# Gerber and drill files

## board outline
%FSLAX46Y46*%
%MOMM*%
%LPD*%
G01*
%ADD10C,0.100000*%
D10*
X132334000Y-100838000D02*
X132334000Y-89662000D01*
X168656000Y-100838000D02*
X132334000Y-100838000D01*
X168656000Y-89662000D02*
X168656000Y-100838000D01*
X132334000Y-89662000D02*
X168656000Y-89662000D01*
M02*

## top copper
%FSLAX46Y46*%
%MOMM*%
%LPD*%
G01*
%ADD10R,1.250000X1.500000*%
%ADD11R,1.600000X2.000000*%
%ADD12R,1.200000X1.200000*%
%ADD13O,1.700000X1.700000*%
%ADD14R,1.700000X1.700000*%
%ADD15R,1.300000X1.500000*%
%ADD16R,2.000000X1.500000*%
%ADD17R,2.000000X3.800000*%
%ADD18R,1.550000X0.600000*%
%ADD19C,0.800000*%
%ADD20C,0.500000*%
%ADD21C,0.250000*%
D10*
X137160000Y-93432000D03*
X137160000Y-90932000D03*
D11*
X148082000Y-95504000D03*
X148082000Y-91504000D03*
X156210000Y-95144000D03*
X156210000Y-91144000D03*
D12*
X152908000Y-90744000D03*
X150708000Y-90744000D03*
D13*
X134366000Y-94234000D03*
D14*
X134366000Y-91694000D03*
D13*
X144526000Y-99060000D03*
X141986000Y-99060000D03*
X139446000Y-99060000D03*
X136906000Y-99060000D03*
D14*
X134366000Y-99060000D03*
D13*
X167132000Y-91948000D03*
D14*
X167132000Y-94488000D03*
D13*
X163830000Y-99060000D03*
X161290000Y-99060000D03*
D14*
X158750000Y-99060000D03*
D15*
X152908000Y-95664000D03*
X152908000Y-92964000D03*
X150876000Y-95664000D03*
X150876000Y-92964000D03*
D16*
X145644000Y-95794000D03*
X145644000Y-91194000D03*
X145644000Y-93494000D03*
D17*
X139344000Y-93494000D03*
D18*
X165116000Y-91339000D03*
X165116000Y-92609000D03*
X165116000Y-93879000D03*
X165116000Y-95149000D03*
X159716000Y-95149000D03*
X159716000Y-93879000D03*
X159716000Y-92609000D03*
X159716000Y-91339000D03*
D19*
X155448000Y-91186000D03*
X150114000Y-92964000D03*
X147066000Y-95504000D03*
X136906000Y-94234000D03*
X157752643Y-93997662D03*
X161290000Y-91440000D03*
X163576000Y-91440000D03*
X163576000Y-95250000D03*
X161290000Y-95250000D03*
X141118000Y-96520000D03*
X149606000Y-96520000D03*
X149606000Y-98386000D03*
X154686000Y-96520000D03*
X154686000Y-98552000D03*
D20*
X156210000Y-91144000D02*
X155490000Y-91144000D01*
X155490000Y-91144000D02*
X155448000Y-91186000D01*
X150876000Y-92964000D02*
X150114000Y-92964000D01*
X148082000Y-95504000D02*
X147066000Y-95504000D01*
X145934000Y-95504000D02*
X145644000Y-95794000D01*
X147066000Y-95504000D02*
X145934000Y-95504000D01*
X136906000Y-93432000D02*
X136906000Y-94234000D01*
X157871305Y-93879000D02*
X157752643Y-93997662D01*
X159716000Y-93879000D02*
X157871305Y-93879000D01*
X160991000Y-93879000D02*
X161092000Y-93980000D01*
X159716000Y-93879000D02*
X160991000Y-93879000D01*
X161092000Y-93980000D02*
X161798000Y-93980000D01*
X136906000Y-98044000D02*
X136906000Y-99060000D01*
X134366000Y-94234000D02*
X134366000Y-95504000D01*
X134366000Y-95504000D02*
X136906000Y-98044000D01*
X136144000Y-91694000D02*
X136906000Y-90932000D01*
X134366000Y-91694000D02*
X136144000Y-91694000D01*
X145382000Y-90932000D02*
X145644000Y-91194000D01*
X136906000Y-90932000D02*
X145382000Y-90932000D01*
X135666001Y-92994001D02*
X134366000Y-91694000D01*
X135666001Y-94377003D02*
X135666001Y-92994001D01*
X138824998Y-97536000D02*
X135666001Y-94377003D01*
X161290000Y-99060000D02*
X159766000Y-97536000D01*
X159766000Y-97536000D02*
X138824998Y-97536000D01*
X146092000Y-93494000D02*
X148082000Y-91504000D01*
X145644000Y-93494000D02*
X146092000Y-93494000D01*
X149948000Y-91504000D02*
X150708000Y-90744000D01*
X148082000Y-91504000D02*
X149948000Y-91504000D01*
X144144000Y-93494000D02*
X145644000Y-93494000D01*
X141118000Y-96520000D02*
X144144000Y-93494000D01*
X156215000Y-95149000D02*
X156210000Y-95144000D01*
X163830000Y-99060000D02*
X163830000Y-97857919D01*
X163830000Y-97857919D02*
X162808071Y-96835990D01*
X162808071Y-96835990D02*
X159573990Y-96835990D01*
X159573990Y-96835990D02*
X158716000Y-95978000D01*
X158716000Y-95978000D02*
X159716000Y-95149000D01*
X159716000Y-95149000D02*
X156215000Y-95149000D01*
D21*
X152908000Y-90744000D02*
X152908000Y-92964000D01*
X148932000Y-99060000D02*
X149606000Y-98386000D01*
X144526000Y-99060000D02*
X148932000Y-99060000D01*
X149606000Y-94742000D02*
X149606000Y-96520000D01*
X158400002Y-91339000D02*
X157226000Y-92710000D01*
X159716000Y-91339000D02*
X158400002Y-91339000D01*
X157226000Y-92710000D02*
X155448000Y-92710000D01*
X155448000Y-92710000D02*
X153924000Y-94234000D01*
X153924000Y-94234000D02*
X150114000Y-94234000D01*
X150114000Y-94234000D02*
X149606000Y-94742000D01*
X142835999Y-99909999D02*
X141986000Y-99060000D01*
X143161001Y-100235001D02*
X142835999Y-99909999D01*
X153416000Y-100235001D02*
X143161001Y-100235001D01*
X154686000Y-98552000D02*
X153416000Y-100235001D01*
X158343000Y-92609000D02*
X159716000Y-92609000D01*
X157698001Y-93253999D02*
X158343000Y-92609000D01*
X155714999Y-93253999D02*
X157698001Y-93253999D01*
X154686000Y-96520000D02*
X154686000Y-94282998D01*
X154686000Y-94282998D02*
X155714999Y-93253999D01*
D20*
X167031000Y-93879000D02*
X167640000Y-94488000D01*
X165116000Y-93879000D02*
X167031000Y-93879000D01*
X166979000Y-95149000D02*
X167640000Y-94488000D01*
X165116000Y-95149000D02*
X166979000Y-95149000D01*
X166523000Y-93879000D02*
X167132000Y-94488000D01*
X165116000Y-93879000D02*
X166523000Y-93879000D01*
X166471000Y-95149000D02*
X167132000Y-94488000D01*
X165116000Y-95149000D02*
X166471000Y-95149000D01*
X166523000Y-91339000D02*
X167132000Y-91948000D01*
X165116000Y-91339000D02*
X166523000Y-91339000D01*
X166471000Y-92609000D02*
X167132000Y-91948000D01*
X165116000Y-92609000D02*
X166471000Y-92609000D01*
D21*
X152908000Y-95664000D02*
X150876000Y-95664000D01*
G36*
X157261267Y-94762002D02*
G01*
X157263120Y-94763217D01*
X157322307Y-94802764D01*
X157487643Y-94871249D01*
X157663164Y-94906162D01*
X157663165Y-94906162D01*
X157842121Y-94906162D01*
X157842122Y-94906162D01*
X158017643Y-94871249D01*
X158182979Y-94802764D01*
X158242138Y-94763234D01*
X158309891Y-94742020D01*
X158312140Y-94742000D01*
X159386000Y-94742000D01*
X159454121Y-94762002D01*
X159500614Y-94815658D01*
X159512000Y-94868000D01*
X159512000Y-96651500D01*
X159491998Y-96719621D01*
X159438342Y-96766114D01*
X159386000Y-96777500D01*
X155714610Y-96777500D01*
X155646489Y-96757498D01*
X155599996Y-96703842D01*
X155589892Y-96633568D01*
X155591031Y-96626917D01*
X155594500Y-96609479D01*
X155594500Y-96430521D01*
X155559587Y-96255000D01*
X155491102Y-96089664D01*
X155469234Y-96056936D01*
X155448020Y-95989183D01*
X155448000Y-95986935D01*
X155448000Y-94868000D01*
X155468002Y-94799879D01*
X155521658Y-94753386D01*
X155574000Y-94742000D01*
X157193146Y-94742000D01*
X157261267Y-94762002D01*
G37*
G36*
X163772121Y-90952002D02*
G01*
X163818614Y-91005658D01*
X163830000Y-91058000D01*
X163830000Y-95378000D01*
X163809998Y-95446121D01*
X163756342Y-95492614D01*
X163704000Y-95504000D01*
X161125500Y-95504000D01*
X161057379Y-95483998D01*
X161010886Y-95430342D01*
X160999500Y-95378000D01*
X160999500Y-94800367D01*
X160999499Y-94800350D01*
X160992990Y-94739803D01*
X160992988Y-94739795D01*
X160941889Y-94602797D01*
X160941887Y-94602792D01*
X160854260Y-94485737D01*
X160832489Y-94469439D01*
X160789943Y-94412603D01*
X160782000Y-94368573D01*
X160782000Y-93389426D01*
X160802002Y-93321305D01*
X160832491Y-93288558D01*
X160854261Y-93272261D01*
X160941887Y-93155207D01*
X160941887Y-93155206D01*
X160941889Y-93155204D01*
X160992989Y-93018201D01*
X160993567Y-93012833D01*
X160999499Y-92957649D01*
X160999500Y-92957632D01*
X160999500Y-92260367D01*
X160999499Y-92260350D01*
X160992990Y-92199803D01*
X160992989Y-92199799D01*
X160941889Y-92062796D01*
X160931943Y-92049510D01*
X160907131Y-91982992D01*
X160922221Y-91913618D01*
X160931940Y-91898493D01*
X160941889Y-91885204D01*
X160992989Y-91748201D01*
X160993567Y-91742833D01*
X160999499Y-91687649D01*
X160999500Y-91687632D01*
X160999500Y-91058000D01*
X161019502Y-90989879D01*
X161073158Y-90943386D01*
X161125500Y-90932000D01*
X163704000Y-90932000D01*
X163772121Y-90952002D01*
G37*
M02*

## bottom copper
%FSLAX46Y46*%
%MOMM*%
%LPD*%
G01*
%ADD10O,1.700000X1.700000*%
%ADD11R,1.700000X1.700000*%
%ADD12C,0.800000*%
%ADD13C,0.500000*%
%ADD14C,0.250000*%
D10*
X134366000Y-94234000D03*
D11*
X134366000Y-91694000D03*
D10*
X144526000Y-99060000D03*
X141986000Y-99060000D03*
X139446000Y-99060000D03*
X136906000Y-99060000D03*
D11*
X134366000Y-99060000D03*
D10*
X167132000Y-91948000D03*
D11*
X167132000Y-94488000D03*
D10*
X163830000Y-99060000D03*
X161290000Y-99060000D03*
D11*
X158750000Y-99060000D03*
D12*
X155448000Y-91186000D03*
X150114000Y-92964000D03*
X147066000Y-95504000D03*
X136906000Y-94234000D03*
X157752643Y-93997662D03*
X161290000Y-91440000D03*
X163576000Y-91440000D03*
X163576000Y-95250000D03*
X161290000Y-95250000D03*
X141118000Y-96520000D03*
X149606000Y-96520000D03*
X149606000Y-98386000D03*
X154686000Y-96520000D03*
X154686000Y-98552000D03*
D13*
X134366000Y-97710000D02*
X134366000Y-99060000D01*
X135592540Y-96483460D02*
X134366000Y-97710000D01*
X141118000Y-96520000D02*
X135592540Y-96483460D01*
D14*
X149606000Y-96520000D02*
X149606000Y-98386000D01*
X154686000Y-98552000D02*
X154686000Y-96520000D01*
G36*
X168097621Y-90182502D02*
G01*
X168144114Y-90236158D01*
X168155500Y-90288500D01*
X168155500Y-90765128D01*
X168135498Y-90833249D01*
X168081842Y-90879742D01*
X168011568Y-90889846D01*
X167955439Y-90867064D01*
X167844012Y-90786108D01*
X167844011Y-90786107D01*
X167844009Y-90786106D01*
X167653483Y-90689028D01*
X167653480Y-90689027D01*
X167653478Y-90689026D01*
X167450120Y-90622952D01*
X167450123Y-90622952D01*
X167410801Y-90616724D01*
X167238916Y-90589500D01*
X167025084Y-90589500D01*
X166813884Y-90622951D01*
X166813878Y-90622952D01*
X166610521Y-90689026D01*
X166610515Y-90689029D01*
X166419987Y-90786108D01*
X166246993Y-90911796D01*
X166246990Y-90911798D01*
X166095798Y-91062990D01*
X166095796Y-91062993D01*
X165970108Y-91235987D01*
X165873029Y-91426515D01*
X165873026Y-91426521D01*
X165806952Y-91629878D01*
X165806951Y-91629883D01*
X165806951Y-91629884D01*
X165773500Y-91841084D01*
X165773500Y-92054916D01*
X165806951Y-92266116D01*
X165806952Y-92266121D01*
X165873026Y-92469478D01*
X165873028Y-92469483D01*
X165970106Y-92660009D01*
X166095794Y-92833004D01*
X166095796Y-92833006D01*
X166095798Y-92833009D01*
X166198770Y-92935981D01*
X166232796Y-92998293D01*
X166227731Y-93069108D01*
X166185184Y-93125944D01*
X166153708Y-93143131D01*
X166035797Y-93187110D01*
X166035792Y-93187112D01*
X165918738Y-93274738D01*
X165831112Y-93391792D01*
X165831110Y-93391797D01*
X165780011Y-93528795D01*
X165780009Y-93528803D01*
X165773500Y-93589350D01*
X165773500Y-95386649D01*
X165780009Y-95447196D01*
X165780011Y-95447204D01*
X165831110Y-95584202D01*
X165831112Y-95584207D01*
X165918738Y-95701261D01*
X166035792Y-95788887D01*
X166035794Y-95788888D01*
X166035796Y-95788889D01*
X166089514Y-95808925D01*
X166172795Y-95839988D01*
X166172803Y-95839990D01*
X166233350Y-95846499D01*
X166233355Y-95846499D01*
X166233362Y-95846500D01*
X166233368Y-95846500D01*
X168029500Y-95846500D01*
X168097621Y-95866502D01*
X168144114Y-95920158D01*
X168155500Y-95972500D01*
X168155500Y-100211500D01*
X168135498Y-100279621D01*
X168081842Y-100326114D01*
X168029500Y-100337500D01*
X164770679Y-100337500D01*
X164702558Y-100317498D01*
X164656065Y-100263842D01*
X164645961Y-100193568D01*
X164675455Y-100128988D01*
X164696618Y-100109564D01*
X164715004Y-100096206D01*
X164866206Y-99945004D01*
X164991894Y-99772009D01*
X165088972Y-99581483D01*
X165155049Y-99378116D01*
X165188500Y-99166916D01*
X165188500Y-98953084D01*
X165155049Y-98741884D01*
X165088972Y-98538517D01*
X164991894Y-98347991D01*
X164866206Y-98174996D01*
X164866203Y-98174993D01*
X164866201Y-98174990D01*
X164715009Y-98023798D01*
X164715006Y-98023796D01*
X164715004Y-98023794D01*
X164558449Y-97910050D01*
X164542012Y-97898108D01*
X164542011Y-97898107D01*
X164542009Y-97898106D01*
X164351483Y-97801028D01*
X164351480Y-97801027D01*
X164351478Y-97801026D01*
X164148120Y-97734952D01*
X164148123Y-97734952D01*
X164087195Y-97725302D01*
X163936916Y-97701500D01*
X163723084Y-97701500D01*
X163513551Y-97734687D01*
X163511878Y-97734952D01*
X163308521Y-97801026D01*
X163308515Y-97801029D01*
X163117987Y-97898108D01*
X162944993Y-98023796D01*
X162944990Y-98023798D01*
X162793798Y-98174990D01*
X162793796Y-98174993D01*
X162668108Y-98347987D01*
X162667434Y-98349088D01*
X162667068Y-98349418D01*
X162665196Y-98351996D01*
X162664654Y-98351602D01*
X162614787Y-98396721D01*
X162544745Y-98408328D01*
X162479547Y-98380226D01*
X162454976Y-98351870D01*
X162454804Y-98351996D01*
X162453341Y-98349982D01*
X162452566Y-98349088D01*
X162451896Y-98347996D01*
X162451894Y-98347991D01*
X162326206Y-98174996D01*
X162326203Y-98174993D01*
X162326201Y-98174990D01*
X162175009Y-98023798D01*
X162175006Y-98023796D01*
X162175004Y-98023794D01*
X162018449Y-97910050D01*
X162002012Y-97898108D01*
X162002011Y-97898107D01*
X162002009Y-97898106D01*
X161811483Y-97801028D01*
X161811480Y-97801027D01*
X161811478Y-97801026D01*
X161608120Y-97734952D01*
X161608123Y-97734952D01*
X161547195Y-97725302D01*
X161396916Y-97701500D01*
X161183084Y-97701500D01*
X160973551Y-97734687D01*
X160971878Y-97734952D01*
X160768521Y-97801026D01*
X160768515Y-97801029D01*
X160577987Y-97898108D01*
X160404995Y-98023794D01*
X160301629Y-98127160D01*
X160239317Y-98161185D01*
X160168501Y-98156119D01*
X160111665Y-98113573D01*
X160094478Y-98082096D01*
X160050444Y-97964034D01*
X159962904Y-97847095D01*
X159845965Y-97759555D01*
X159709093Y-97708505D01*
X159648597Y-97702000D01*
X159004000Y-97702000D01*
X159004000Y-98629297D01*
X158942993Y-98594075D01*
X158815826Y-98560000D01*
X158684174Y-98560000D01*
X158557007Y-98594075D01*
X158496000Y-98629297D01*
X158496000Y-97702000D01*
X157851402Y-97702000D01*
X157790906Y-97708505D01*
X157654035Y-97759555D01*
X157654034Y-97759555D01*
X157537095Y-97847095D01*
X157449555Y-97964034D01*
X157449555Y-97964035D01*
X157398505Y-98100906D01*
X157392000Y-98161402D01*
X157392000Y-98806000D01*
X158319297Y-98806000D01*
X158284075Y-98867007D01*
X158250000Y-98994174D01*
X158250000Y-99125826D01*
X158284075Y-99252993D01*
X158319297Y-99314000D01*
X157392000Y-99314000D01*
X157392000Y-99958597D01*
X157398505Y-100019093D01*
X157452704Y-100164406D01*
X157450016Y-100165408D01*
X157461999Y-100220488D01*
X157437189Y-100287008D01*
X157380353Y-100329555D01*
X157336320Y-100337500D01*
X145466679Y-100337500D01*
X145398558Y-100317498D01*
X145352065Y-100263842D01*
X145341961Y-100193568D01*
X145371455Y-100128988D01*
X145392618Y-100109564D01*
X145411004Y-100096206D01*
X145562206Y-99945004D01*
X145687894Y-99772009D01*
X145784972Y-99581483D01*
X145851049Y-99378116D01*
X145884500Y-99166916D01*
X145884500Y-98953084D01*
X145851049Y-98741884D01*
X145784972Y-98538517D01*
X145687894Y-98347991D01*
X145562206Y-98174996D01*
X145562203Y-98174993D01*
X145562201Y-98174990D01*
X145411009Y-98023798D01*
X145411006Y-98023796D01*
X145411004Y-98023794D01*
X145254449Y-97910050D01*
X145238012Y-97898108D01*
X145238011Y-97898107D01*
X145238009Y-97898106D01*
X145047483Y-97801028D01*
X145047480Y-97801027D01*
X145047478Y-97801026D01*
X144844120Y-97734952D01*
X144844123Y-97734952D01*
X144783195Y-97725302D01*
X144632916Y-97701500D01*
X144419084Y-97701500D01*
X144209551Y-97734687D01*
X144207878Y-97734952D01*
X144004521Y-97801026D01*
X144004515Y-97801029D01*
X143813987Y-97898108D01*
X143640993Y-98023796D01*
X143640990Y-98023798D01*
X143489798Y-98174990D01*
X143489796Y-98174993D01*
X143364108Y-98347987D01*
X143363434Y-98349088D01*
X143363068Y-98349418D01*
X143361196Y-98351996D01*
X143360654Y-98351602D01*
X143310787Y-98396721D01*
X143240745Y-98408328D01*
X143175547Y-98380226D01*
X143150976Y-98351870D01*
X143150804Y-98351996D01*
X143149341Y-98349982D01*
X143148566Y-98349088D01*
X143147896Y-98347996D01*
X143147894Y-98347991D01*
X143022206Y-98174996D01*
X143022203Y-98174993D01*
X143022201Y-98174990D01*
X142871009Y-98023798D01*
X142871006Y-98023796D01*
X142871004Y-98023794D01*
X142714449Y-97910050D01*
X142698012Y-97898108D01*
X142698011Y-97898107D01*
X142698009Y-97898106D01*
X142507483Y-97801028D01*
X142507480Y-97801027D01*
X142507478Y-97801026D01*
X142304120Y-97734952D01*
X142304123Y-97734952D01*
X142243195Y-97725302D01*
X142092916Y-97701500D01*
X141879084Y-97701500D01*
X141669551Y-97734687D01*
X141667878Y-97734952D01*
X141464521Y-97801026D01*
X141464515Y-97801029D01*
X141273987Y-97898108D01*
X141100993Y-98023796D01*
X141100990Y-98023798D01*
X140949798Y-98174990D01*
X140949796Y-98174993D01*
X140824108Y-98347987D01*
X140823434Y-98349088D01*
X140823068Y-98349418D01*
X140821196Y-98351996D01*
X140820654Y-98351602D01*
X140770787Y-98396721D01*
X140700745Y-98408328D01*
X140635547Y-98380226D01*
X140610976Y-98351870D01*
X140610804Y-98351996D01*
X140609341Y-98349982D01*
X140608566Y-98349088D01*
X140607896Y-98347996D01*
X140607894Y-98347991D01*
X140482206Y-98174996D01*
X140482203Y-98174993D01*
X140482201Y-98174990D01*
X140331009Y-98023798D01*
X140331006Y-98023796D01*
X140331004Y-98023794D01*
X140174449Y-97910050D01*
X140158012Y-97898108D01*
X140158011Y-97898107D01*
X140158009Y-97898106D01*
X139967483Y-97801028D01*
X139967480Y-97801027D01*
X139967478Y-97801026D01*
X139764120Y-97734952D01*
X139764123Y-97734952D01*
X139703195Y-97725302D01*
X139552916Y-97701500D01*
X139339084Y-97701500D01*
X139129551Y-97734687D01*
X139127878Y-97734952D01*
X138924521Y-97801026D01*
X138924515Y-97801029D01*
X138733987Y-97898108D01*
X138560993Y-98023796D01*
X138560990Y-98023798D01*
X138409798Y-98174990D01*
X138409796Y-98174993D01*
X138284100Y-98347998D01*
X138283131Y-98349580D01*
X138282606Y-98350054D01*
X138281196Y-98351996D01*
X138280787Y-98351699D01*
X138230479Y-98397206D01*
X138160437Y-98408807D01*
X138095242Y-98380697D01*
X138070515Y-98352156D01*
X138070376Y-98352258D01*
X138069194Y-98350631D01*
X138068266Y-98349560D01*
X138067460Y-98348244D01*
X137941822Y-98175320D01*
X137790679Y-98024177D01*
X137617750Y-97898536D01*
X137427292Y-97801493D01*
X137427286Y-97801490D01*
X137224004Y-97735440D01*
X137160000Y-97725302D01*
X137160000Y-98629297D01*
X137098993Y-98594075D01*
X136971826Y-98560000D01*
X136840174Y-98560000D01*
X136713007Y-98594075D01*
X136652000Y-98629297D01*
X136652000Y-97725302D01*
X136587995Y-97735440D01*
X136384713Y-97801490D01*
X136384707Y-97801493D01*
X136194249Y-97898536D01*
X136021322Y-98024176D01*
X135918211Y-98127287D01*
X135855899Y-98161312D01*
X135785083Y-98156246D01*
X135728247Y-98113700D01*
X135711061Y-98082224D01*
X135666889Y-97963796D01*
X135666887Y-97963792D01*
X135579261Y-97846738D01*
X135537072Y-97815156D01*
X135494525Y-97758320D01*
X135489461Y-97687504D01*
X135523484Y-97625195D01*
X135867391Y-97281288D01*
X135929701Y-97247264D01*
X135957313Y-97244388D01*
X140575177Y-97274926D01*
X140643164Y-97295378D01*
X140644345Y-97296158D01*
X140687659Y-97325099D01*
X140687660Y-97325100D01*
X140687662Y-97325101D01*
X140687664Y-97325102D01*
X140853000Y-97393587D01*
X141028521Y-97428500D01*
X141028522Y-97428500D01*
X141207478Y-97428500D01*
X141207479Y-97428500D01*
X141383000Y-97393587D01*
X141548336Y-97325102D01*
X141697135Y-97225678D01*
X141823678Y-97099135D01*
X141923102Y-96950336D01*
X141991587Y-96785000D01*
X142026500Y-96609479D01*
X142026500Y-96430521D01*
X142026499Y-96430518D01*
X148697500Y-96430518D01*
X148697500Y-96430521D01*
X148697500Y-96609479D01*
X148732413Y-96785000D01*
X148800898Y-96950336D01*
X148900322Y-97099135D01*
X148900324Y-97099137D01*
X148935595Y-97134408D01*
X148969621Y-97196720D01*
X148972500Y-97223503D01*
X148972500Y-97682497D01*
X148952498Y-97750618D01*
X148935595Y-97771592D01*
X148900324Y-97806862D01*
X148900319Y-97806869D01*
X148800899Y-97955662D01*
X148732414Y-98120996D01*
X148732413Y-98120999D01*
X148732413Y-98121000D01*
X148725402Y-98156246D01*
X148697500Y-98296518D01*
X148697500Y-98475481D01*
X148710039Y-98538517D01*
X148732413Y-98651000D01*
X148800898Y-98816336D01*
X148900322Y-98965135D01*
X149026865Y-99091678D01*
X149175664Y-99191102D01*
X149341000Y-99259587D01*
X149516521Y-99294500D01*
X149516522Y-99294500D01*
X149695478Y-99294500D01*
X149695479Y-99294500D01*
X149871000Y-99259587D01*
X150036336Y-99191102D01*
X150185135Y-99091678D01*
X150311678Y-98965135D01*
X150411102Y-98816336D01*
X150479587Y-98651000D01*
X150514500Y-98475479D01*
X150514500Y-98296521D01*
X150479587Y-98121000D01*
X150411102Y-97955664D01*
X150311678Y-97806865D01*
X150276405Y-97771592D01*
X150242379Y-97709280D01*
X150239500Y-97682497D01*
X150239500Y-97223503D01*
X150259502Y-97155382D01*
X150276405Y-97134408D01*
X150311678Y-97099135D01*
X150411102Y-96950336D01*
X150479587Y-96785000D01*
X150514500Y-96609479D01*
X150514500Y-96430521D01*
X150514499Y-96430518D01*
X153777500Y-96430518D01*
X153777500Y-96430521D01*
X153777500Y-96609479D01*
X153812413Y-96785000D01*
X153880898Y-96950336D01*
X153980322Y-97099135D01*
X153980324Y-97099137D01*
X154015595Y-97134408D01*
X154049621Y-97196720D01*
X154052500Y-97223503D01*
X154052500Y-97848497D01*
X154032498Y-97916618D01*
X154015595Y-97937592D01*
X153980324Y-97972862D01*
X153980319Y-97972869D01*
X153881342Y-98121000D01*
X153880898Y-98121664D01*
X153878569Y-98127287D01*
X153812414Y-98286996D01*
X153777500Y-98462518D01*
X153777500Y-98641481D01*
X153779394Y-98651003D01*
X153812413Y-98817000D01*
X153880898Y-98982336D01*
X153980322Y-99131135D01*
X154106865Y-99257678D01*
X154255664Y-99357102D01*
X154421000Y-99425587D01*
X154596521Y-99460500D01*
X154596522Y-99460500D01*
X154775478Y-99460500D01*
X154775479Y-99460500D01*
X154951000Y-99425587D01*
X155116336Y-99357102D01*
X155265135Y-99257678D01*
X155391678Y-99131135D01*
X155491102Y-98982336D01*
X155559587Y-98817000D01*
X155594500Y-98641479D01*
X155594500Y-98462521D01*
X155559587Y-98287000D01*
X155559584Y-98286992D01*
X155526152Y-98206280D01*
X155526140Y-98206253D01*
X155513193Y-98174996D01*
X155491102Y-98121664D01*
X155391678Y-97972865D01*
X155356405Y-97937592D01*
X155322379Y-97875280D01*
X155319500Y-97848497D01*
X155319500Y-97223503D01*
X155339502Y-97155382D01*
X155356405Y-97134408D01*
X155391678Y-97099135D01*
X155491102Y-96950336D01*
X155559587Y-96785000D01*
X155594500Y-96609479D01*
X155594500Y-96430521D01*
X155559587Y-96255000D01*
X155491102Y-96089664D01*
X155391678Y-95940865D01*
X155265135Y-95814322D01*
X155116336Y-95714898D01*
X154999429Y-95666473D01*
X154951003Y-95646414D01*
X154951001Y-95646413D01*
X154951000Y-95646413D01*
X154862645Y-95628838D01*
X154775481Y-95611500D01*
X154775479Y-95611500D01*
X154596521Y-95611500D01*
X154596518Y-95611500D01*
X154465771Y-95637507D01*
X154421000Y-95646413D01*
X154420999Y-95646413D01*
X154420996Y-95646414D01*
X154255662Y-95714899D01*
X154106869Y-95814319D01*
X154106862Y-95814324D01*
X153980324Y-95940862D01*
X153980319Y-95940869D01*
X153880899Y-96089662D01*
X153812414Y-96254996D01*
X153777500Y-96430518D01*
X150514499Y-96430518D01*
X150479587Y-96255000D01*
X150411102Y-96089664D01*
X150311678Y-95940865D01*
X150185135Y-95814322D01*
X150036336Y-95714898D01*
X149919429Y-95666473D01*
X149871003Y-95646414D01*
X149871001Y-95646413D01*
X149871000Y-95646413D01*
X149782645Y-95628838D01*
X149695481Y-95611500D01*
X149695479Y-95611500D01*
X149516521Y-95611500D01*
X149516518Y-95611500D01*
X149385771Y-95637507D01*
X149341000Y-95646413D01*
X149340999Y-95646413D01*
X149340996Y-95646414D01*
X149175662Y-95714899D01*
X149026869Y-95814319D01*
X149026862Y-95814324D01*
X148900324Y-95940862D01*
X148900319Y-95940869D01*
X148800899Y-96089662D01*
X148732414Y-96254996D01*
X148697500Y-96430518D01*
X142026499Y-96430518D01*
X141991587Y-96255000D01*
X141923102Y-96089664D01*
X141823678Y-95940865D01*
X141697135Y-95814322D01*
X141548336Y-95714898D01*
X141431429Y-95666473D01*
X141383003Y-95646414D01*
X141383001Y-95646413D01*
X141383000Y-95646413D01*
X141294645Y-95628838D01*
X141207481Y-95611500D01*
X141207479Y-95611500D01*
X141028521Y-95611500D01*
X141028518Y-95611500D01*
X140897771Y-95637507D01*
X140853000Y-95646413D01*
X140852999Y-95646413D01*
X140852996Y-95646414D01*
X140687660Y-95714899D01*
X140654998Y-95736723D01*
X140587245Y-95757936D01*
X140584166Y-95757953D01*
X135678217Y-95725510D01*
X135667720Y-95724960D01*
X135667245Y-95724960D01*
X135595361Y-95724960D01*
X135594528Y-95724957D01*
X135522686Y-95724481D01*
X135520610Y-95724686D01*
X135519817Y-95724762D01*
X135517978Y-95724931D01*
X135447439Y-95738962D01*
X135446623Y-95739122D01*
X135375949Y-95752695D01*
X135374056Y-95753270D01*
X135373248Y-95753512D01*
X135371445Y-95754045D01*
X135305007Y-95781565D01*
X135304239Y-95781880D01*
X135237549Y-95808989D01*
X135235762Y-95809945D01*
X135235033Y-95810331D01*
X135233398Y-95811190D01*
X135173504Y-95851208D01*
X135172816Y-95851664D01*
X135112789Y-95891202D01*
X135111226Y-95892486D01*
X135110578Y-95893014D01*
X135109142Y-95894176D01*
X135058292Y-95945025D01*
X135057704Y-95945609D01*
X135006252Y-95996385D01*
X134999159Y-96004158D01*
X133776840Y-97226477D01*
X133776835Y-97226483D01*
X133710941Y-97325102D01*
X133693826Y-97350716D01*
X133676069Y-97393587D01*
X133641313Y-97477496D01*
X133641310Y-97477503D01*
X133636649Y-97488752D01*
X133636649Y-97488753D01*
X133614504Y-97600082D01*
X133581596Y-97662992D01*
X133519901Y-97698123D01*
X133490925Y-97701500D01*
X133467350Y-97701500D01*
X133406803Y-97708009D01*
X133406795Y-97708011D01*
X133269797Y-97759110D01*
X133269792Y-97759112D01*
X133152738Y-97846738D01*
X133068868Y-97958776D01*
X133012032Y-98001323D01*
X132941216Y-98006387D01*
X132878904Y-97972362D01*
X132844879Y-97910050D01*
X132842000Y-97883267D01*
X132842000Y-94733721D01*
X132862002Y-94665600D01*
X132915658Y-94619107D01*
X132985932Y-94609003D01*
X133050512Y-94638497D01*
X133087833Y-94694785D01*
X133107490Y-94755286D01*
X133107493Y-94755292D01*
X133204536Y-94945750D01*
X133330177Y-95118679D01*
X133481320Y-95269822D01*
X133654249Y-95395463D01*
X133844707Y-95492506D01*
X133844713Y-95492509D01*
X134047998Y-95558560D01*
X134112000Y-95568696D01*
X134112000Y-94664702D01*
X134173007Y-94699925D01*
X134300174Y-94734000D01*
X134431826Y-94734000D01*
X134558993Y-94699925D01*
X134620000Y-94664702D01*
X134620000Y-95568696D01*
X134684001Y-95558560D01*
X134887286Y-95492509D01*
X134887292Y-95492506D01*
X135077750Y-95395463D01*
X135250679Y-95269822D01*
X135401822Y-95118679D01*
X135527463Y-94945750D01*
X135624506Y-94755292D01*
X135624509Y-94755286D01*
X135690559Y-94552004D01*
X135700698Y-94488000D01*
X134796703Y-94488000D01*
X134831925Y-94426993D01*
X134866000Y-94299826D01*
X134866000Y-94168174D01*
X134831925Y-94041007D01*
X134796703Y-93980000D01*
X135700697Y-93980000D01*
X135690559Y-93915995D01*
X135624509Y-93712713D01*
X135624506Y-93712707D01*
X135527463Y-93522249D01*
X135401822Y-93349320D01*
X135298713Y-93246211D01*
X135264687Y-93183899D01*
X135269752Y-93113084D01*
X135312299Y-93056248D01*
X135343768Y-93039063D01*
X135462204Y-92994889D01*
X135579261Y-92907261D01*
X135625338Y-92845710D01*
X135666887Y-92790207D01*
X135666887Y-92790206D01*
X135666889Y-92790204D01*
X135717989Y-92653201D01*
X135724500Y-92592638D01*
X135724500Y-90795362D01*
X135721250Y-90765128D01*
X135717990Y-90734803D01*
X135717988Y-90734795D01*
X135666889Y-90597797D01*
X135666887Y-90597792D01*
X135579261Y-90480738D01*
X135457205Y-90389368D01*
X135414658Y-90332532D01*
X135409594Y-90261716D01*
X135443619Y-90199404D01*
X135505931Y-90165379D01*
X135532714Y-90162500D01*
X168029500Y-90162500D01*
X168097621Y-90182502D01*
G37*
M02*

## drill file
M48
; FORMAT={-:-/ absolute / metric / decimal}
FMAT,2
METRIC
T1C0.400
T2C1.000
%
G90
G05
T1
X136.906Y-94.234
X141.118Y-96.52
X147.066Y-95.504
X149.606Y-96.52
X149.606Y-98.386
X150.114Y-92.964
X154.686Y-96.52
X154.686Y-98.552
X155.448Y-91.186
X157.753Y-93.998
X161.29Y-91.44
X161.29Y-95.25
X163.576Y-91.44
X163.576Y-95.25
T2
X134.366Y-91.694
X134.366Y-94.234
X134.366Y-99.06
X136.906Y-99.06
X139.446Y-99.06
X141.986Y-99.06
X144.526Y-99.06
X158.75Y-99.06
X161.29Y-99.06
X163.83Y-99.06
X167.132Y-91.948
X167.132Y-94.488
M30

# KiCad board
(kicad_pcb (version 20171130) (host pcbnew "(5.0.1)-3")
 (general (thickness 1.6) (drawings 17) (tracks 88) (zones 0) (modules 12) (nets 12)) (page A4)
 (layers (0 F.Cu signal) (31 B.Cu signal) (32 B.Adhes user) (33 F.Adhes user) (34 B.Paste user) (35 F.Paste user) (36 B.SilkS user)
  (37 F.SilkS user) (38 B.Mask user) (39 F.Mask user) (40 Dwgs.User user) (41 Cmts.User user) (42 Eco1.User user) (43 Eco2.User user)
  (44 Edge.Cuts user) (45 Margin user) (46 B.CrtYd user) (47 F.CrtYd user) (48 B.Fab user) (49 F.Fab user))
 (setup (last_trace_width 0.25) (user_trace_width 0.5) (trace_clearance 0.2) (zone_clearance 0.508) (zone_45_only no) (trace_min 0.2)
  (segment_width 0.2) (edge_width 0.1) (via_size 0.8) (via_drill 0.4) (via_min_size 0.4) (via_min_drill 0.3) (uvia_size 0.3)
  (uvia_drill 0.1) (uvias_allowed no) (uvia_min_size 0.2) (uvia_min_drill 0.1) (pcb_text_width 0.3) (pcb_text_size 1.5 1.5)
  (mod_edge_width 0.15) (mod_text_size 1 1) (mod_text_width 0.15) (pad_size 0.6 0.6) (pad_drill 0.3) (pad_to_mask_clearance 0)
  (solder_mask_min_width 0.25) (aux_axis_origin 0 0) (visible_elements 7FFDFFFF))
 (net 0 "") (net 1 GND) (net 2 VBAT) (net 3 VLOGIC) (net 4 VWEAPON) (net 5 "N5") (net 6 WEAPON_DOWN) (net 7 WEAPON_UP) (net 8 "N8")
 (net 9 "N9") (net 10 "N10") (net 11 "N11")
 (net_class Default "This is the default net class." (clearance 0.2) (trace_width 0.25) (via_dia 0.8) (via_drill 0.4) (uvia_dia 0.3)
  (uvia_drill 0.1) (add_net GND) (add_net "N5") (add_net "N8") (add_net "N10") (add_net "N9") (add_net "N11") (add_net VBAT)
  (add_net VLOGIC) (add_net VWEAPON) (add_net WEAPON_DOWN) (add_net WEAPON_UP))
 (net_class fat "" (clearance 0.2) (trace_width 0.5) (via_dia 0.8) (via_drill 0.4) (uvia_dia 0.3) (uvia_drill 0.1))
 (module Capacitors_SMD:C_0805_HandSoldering (layer F.Cu) (at 137.16 92.182 270)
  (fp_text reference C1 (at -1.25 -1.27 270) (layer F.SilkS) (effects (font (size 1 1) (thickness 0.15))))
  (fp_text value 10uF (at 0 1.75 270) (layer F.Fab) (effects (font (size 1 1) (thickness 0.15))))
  (pad 2 smd rect (at 1.25 0 270) (size 1.5 1.25) (layers F.Cu F.Paste F.Mask) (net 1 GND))
  (pad 1 smd rect (at -1.25 0 270) (size 1.5 1.25) (layers F.Cu F.Paste F.Mask) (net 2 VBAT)))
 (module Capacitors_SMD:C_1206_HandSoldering (layer F.Cu) (at 148.082 93.504 270)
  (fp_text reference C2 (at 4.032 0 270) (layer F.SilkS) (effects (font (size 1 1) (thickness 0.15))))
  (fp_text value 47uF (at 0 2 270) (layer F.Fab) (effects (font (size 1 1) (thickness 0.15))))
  (pad 2 smd rect (at 2 0 270) (size 2 1.6) (layers F.Cu F.Paste F.Mask) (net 1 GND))
  (pad 1 smd rect (at -2 0 270) (size 2 1.6) (layers F.Cu F.Paste F.Mask) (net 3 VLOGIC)))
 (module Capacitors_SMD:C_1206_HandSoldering (layer F.Cu) (at 156.21 93.144 90)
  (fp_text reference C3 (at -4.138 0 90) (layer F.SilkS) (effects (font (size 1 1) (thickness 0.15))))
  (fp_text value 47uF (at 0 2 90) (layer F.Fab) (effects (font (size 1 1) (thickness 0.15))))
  (pad 1 smd rect (at -2 0 90) (size 2 1.6) (layers F.Cu F.Paste F.Mask) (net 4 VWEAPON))
  (pad 2 smd rect (at 2 0 90) (size 2 1.6) (layers F.Cu F.Paste F.Mask) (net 1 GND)))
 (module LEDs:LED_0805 (layer F.Cu) (at 151.808 90.744 180)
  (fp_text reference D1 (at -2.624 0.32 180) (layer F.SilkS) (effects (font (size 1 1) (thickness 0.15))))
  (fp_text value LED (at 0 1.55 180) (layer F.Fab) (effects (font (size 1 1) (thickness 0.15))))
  (pad 1 smd rect (at -1.1 0) (size 1.2 1.2) (layers F.Cu F.Paste F.Mask) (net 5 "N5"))
  (pad 2 smd rect (at 1.1 0) (size 1.2 1.2) (layers F.Cu F.Paste F.Mask) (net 3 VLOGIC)))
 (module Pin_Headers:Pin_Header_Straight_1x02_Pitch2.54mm (layer F.Cu) (at 134.366 91.694)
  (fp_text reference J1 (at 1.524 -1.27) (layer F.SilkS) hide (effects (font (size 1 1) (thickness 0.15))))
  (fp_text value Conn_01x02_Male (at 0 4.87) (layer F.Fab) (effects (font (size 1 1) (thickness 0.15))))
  (pad 2 thru_hole oval (at 0 2.54) (size 1.7 1.7) (drill 1) (layers *.Cu *.Mask) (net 1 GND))
  (pad 1 thru_hole rect (at 0 0) (size 1.7 1.7) (drill 1) (layers *.Cu *.Mask) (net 2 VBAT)))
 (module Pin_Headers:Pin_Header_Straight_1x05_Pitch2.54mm (layer F.Cu) (at 134.366 99.06 90)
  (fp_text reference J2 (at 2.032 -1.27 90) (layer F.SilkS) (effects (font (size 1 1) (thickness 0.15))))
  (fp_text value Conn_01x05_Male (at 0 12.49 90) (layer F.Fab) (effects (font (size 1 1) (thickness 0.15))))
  (pad 5 thru_hole oval (at 0 10.16 90) (size 1.7 1.7) (drill 1) (layers *.Cu *.Mask) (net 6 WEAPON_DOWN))
  (pad 4 thru_hole oval (at 0 7.62 90) (size 1.7 1.7) (drill 1) (layers *.Cu *.Mask) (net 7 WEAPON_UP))
  (pad 3 thru_hole oval (at 0 5.08 90) (size 1.7 1.7) (drill 1) (layers *.Cu *.Mask) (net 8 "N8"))
  (pad 2 thru_hole oval (at 0 2.54 90) (size 1.7 1.7) (drill 1) (layers *.Cu *.Mask) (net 1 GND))
  (pad 1 thru_hole rect (at 0 0 90) (size 1.7 1.7) (drill 1) (layers *.Cu *.Mask) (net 3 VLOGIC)))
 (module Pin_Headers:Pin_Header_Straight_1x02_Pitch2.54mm (layer F.Cu) (at 167.132 94.488 180)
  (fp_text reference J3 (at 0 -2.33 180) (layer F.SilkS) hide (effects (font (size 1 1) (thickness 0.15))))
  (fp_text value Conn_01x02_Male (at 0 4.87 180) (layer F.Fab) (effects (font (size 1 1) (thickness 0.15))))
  (pad 2 thru_hole oval (at 0 2.54 180) (size 1.7 1.7) (drill 1) (layers *.Cu *.Mask) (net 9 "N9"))
  (pad 1 thru_hole rect (at 0 0 180) (size 1.7 1.7) (drill 1) (layers *.Cu *.Mask) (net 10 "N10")))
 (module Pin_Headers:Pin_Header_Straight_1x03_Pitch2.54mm (layer F.Cu) (at 158.75 99.06 90)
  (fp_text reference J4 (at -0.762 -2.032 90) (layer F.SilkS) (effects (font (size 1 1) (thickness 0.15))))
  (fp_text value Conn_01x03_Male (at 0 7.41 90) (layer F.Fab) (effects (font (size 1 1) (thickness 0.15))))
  (pad 3 thru_hole oval (at 0 5.08 90) (size 1.7 1.7) (drill 1) (layers *.Cu *.Mask) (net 4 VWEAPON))
  (pad 2 thru_hole oval (at 0 2.54 90) (size 1.7 1.7) (drill 1) (layers *.Cu *.Mask) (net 2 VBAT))
  (pad 1 thru_hole rect (at 0 0 90) (size 1.7 1.7) (drill 1) (layers *.Cu *.Mask) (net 1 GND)))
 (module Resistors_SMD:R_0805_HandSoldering (layer F.Cu) (at 152.908 94.314 270)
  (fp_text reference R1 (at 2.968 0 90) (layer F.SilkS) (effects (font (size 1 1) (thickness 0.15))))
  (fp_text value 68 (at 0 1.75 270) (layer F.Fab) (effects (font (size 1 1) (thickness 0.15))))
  (pad 2 smd rect (at 1.35 0 270) (size 1.5 1.3) (layers F.Cu F.Paste F.Mask) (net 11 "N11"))
  (pad 1 smd rect (at -1.35 0 270) (size 1.5 1.3) (layers F.Cu F.Paste F.Mask) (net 5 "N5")))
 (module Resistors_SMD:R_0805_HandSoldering (layer F.Cu) (at 150.876 94.314 90)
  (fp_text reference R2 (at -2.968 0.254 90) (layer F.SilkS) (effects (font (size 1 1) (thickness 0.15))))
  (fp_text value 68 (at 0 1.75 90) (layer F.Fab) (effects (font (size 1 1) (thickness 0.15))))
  (pad 1 smd rect (at -1.35 0 90) (size 1.5 1.3) (layers F.Cu F.Paste F.Mask) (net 11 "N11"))
  (pad 2 smd rect (at 1.35 0 90) (size 1.5 1.3) (layers F.Cu F.Paste F.Mask) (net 1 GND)))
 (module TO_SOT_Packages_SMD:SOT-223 (layer F.Cu) (at 142.494 93.494 180)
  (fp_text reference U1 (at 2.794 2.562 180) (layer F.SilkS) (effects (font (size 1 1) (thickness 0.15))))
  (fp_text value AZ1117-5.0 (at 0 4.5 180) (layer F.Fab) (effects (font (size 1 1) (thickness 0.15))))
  (pad 1 smd rect (at -3.15 -2.3 180) (size 2 1.5) (layers F.Cu F.Paste F.Mask) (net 1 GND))
  (pad 3 smd rect (at -3.15 2.3 180) (size 2 1.5) (layers F.Cu F.Paste F.Mask) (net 2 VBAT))
  (pad 2 smd rect (at -3.15 0 180) (size 2 1.5) (layers F.Cu F.Paste F.Mask) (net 3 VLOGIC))
  (pad 4 smd rect (at 3.15 0 180) (size 2 3.8) (layers F.Cu F.Paste F.Mask)))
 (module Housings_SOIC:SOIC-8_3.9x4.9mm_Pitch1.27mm (layer F.Cu) (at 162.416 93.244)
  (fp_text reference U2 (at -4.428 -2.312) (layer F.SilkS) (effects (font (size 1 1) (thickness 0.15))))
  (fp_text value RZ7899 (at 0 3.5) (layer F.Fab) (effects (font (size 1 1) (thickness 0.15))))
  (pad 8 smd rect (at 2.7 -1.905) (size 1.55 0.6) (layers F.Cu F.Paste F.Mask) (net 9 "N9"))
  (pad 7 smd rect (at 2.7 -0.635) (size 1.55 0.6) (layers F.Cu F.Paste F.Mask) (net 9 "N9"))
  (pad 6 smd rect (at 2.7 0.635) (size 1.55 0.6) (layers F.Cu F.Paste F.Mask) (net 10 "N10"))
  (pad 5 smd rect (at 2.7 1.905) (size 1.55 0.6) (layers F.Cu F.Paste F.Mask) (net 10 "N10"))
  (pad 4 smd rect (at -2.7 1.905) (size 1.55 0.6) (layers F.Cu F.Paste F.Mask) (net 4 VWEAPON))
  (pad 3 smd rect (at -2.7 0.635) (size 1.55 0.6) (layers F.Cu F.Paste F.Mask) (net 1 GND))
  (pad 2 smd rect (at -2.7 -0.635) (size 1.55 0.6) (layers F.Cu F.Paste F.Mask) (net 7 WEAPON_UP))
  (pad 1 smd rect (at -2.7 -1.905) (size 1.55 0.6) (layers F.Cu F.Paste F.Mask) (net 6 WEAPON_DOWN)))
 (gr_line (start 132.334 100.838) (end 132.334 89.662) (layer Edge.Cuts) (width 0.1))
 (gr_line (start 168.656 100.838) (end 132.334 100.838) (layer Edge.Cuts) (width 0.1))
 (gr_line (start 168.656 89.662) (end 168.656 100.838) (layer Edge.Cuts) (width 0.1))
 (gr_line (start 132.334 89.662) (end 168.656 89.662) (layer Edge.Cuts) (width 0.1))
 (via (at 155.448 91.186) (size 0.8) (drill 0.4) (layers F.Cu B.Cu) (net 1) (status 30))
 (segment (start 156.21 91.144) (end 155.49 91.144) (width 0.5) (layer F.Cu) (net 1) (status 30))
 (segment (start 155.49 91.144) (end 155.448 91.186) (width 0.5) (layer F.Cu) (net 1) (status 30))
 (via (at 150.114 92.964) (size 0.8) (drill 0.4) (layers F.Cu B.Cu) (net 1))
 (segment (start 150.876 92.964) (end 150.114 92.964) (width 0.5) (layer F.Cu) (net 1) (status 10))
 (via (at 147.066 95.504) (size 0.8) (drill 0.4) (layers F.Cu B.Cu) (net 1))
 (segment (start 148.082 95.504) (end 147.066 95.504) (width 0.5) (layer F.Cu) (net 1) (status 10))
 (segment (start 145.934 95.504) (end 145.644 95.794) (width 0.5) (layer F.Cu) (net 1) (status 30))
 (segment (start 147.066 95.504) (end 145.934 95.504) (width 0.5) (layer F.Cu) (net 1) (status 20))
 (via (at 136.906 94.234) (size 0.8) (drill 0.4) (layers F.Cu B.Cu) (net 1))
 (segment (start 136.906 93.432) (end 136.906 94.234) (width 0.5) (layer F.Cu) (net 1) (status 10))
 (via (at 157.752643 93.997662) (size 0.8) (drill 0.4) (layers F.Cu B.Cu) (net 1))
 (segment (start 157.871305 93.879) (end 157.752643 93.997662) (width 0.5) (layer F.Cu) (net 1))
 (segment (start 159.716 93.879) (end 157.871305 93.879) (width 0.5) (layer F.Cu) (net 1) (status 10))
 (segment (start 160.991 93.879) (end 161.092 93.98) (width 0.5) (layer F.Cu) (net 1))
 (segment (start 159.716 93.879) (end 160.991 93.879) (width 0.5) (layer F.Cu) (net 1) (status 10))
 (segment (start 161.092 93.98) (end 161.798 93.98) (width 0.5) (layer F.Cu) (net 1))
 (via (at 161.29 91.44) (size 0.8) (drill 0.4) (layers F.Cu B.Cu) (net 1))
 (via (at 163.576 91.44) (size 0.8) (drill 0.4) (layers F.Cu B.Cu) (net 1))
 (via (at 163.576 95.25) (size 0.8) (drill 0.4) (layers F.Cu B.Cu) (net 1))
 (via (at 161.29 95.25) (size 0.8) (drill 0.4) (layers F.Cu B.Cu) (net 1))
 (segment (start 136.906 98.044) (end 136.906 99.06) (width 0.5) (layer F.Cu) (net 1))
 (segment (start 134.366 94.234) (end 134.366 95.504) (width 0.5) (layer F.Cu) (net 1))
 (segment (start 134.366 95.504) (end 136.906 98.044) (width 0.5) (layer F.Cu) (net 1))
 (segment (start 136.144 91.694) (end 136.906 90.932) (width 0.5) (layer F.Cu) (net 2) (status 20))
 (segment (start 134.366 91.694) (end 136.144 91.694) (width 0.5) (layer F.Cu) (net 2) (status 10))
 (segment (start 145.382 90.932) (end 145.644 91.194) (width 0.5) (layer F.Cu) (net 2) (status 30))
 (segment (start 136.906 90.932) (end 145.382 90.932) (width 0.5) (layer F.Cu) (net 2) (status 30))
 (segment (start 135.666001 92.994001) (end 134.366 91.694) (width 0.5) (layer F.Cu) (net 2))
 (segment (start 135.666001 94.377003) (end 135.666001 92.994001) (width 0.5) (layer F.Cu) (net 2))
 (segment (start 138.824998 97.536) (end 135.666001 94.377003) (width 0.5) (layer F.Cu) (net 2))
 (segment (start 161.29 99.06) (end 159.766 97.536) (width 0.5) (layer F.Cu) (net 2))
 (segment (start 159.766 97.536) (end 138.824998 97.536) (width 0.5) (layer F.Cu) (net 2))
 (segment (start 146.092 93.494) (end 148.082 91.504) (width 0.5) (layer F.Cu) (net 3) (status 30))
 (segment (start 145.644 93.494) (end 146.092 93.494) (width 0.5) (layer F.Cu) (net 3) (status 30))
 (segment (start 149.948 91.504) (end 150.708 90.744) (width 0.5) (layer F.Cu) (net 3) (status 20))
 (segment (start 148.082 91.504) (end 149.948 91.504) (width 0.5) (layer F.Cu) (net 3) (status 10))
 (segment (start 134.366 97.71) (end 134.366 99.06) (width 0.5) (layer B.Cu) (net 3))
 (segment (start 135.59254 96.48346) (end 134.366 97.71) (width 0.5) (layer B.Cu) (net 3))
 (segment (start 141.118 96.52) (end 135.59254 96.48346) (width 0.5) (layer B.Cu) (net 3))
 (via (at 141.118 96.52) (size 0.8) (drill 0.4) (layers F.Cu B.Cu) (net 3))
 (segment (start 144.144 93.494) (end 145.644 93.494) (width 0.5) (layer F.Cu) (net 3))
 (segment (start 141.118 96.52) (end 144.144 93.494) (width 0.5) (layer F.Cu) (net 3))
 (segment (start 156.215 95.149) (end 156.21 95.144) (width 0.5) (layer F.Cu) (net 4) (status 30))
 (segment (start 163.83 99.06) (end 163.83 97.857919) (width 0.5) (layer F.Cu) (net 4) (status 10))
 (segment (start 163.83 97.857919) (end 162.808071 96.83599) (width 0.5) (layer F.Cu) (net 4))
 (segment (start 162.808071 96.83599) (end 159.57399 96.83599) (width 0.5) (layer F.Cu) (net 4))
 (segment (start 159.57399 96.83599) (end 158.716 95.978) (width 0.5) (layer F.Cu) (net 4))
 (segment (start 158.716 95.978) (end 159.716 95.149) (width 0.5) (layer F.Cu) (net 4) (status 20))
 (segment (start 159.716 95.149) (end 156.215 95.149) (width 0.5) (layer F.Cu) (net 4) (status 30))
 (segment (start 152.908 90.744) (end 152.908 92.964) (width 0.25) (layer F.Cu) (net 5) (status 30))
 (via (at 149.606 96.52) (size 0.8) (drill 0.4) (layers F.Cu B.Cu) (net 6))
 (via (at 149.606 98.386) (size 0.8) (drill 0.4) (layers F.Cu B.Cu) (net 6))
 (segment (start 149.606 96.52) (end 149.606 98.386) (width 0.25) (layer B.Cu) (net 6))
 (segment (start 148.932 99.06) (end 149.606 98.386) (width 0.25) (layer F.Cu) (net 6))
 (segment (start 144.526 99.06) (end 148.932 99.06) (width 0.25) (layer F.Cu) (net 6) (status 10))
 (segment (start 149.606 94.742) (end 149.606 96.52) (width 0.25) (layer F.Cu) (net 6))
 (segment (start 158.400002 91.339) (end 157.226 92.71) (width 0.25) (layer F.Cu) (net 6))
 (segment (start 159.716 91.339) (end 158.400002 91.339) (width 0.25) (layer F.Cu) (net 6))
 (segment (start 157.226 92.71) (end 155.448 92.71) (width 0.25) (layer F.Cu) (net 6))
 (segment (start 155.448 92.71) (end 153.924 94.234) (width 0.25) (layer F.Cu) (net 6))
 (segment (start 153.924 94.234) (end 150.114 94.234) (width 0.25) (layer F.Cu) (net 6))
 (segment (start 150.114 94.234) (end 149.606 94.742) (width 0.25) (layer F.Cu) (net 6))
 (segment (start 142.835999 99.909999) (end 141.986 99.06) (width 0.25) (layer F.Cu) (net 7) (status 30))
 (segment (start 143.161001 100.235001) (end 142.835999 99.909999) (width 0.25) (layer F.Cu) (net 7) (status 20))
 (via (at 154.686 96.52) (size 0.8) (drill 0.4) (layers F.Cu B.Cu) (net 7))
 (segment (start 153.416 100.235001) (end 143.161001 100.235001) (width 0.25) (layer F.Cu) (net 7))
 (via (at 154.686 98.552) (size 0.8) (drill 0.4) (layers F.Cu B.Cu) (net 7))
 (segment (start 154.686 98.552) (end 154.686 96.52) (width 0.25) (layer B.Cu) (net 7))
 (segment (start 154.686 98.552) (end 153.416 100.235001) (width 0.25) (layer F.Cu) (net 7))
 (segment (start 158.343 92.609) (end 159.716 92.609) (width 0.25) (layer F.Cu) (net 7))
 (segment (start 157.698001 93.253999) (end 158.343 92.609) (width 0.25) (layer F.Cu) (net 7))
 (segment (start 155.714999 93.253999) (end 157.698001 93.253999) (width 0.25) (layer F.Cu) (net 7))
 (segment (start 154.686 96.52) (end 154.686 94.282998) (width 0.25) (layer F.Cu) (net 7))
 (segment (start 154.686 94.282998) (end 155.714999 93.253999) (width 0.25) (layer F.Cu) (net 7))
 (segment (start 167.031 93.879) (end 167.64 94.488) (width 0.5) (layer F.Cu) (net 10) (status 30))
 (segment (start 165.116 93.879) (end 167.031 93.879) (width 0.5) (layer F.Cu) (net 10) (status 30))
 (segment (start 166.979 95.149) (end 167.64 94.488) (width 0.5) (layer F.Cu) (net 10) (status 30))
 (segment (start 165.116 95.149) (end 166.979 95.149) (width 0.5) (layer F.Cu) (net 10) (status 30))
 (segment (start 166.523 93.879) (end 167.132 94.488) (width 0.5) (layer F.Cu) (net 10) (status 30))
 (segment (start 165.116 93.879) (end 166.523 93.879) (width 0.5) (layer F.Cu) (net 10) (status 30))
 (segment (start 166.471 95.149) (end 167.132 94.488) (width 0.5) (layer F.Cu) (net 10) (status 30))
 (segment (start 165.116 95.149) (end 166.471 95.149) (width 0.5) (layer F.Cu) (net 10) (status 30))
 (segment (start 166.523 91.339) (end 167.132 91.948) (width 0.5) (layer F.Cu) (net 9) (status 30))
 (segment (start 165.116 91.339) (end 166.523 91.339) (width 0.5) (layer F.Cu) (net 9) (status 30))
 (segment (start 166.471 92.609) (end 167.132 91.948) (width 0.5) (layer F.Cu) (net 9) (status 30))
 (segment (start 165.116 92.609) (end 166.471 92.609) (width 0.5) (layer F.Cu) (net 9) (status 30))
 (segment (start 152.908 95.664) (end 150.876 95.664) (width 0.25) (layer F.Cu) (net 11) (status 30))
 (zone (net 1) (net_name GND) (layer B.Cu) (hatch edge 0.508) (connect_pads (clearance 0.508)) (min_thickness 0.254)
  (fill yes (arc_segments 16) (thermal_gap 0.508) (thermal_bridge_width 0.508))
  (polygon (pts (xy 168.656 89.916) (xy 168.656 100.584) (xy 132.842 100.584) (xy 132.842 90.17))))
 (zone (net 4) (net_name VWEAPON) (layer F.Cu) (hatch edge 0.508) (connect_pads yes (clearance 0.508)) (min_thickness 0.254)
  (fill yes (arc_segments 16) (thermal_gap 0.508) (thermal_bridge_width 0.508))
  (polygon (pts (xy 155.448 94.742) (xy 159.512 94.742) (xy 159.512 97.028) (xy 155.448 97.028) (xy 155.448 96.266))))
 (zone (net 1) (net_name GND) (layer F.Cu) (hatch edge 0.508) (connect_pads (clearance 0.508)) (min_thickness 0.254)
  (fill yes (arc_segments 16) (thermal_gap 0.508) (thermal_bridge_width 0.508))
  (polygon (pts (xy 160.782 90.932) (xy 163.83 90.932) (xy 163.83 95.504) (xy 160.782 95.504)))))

